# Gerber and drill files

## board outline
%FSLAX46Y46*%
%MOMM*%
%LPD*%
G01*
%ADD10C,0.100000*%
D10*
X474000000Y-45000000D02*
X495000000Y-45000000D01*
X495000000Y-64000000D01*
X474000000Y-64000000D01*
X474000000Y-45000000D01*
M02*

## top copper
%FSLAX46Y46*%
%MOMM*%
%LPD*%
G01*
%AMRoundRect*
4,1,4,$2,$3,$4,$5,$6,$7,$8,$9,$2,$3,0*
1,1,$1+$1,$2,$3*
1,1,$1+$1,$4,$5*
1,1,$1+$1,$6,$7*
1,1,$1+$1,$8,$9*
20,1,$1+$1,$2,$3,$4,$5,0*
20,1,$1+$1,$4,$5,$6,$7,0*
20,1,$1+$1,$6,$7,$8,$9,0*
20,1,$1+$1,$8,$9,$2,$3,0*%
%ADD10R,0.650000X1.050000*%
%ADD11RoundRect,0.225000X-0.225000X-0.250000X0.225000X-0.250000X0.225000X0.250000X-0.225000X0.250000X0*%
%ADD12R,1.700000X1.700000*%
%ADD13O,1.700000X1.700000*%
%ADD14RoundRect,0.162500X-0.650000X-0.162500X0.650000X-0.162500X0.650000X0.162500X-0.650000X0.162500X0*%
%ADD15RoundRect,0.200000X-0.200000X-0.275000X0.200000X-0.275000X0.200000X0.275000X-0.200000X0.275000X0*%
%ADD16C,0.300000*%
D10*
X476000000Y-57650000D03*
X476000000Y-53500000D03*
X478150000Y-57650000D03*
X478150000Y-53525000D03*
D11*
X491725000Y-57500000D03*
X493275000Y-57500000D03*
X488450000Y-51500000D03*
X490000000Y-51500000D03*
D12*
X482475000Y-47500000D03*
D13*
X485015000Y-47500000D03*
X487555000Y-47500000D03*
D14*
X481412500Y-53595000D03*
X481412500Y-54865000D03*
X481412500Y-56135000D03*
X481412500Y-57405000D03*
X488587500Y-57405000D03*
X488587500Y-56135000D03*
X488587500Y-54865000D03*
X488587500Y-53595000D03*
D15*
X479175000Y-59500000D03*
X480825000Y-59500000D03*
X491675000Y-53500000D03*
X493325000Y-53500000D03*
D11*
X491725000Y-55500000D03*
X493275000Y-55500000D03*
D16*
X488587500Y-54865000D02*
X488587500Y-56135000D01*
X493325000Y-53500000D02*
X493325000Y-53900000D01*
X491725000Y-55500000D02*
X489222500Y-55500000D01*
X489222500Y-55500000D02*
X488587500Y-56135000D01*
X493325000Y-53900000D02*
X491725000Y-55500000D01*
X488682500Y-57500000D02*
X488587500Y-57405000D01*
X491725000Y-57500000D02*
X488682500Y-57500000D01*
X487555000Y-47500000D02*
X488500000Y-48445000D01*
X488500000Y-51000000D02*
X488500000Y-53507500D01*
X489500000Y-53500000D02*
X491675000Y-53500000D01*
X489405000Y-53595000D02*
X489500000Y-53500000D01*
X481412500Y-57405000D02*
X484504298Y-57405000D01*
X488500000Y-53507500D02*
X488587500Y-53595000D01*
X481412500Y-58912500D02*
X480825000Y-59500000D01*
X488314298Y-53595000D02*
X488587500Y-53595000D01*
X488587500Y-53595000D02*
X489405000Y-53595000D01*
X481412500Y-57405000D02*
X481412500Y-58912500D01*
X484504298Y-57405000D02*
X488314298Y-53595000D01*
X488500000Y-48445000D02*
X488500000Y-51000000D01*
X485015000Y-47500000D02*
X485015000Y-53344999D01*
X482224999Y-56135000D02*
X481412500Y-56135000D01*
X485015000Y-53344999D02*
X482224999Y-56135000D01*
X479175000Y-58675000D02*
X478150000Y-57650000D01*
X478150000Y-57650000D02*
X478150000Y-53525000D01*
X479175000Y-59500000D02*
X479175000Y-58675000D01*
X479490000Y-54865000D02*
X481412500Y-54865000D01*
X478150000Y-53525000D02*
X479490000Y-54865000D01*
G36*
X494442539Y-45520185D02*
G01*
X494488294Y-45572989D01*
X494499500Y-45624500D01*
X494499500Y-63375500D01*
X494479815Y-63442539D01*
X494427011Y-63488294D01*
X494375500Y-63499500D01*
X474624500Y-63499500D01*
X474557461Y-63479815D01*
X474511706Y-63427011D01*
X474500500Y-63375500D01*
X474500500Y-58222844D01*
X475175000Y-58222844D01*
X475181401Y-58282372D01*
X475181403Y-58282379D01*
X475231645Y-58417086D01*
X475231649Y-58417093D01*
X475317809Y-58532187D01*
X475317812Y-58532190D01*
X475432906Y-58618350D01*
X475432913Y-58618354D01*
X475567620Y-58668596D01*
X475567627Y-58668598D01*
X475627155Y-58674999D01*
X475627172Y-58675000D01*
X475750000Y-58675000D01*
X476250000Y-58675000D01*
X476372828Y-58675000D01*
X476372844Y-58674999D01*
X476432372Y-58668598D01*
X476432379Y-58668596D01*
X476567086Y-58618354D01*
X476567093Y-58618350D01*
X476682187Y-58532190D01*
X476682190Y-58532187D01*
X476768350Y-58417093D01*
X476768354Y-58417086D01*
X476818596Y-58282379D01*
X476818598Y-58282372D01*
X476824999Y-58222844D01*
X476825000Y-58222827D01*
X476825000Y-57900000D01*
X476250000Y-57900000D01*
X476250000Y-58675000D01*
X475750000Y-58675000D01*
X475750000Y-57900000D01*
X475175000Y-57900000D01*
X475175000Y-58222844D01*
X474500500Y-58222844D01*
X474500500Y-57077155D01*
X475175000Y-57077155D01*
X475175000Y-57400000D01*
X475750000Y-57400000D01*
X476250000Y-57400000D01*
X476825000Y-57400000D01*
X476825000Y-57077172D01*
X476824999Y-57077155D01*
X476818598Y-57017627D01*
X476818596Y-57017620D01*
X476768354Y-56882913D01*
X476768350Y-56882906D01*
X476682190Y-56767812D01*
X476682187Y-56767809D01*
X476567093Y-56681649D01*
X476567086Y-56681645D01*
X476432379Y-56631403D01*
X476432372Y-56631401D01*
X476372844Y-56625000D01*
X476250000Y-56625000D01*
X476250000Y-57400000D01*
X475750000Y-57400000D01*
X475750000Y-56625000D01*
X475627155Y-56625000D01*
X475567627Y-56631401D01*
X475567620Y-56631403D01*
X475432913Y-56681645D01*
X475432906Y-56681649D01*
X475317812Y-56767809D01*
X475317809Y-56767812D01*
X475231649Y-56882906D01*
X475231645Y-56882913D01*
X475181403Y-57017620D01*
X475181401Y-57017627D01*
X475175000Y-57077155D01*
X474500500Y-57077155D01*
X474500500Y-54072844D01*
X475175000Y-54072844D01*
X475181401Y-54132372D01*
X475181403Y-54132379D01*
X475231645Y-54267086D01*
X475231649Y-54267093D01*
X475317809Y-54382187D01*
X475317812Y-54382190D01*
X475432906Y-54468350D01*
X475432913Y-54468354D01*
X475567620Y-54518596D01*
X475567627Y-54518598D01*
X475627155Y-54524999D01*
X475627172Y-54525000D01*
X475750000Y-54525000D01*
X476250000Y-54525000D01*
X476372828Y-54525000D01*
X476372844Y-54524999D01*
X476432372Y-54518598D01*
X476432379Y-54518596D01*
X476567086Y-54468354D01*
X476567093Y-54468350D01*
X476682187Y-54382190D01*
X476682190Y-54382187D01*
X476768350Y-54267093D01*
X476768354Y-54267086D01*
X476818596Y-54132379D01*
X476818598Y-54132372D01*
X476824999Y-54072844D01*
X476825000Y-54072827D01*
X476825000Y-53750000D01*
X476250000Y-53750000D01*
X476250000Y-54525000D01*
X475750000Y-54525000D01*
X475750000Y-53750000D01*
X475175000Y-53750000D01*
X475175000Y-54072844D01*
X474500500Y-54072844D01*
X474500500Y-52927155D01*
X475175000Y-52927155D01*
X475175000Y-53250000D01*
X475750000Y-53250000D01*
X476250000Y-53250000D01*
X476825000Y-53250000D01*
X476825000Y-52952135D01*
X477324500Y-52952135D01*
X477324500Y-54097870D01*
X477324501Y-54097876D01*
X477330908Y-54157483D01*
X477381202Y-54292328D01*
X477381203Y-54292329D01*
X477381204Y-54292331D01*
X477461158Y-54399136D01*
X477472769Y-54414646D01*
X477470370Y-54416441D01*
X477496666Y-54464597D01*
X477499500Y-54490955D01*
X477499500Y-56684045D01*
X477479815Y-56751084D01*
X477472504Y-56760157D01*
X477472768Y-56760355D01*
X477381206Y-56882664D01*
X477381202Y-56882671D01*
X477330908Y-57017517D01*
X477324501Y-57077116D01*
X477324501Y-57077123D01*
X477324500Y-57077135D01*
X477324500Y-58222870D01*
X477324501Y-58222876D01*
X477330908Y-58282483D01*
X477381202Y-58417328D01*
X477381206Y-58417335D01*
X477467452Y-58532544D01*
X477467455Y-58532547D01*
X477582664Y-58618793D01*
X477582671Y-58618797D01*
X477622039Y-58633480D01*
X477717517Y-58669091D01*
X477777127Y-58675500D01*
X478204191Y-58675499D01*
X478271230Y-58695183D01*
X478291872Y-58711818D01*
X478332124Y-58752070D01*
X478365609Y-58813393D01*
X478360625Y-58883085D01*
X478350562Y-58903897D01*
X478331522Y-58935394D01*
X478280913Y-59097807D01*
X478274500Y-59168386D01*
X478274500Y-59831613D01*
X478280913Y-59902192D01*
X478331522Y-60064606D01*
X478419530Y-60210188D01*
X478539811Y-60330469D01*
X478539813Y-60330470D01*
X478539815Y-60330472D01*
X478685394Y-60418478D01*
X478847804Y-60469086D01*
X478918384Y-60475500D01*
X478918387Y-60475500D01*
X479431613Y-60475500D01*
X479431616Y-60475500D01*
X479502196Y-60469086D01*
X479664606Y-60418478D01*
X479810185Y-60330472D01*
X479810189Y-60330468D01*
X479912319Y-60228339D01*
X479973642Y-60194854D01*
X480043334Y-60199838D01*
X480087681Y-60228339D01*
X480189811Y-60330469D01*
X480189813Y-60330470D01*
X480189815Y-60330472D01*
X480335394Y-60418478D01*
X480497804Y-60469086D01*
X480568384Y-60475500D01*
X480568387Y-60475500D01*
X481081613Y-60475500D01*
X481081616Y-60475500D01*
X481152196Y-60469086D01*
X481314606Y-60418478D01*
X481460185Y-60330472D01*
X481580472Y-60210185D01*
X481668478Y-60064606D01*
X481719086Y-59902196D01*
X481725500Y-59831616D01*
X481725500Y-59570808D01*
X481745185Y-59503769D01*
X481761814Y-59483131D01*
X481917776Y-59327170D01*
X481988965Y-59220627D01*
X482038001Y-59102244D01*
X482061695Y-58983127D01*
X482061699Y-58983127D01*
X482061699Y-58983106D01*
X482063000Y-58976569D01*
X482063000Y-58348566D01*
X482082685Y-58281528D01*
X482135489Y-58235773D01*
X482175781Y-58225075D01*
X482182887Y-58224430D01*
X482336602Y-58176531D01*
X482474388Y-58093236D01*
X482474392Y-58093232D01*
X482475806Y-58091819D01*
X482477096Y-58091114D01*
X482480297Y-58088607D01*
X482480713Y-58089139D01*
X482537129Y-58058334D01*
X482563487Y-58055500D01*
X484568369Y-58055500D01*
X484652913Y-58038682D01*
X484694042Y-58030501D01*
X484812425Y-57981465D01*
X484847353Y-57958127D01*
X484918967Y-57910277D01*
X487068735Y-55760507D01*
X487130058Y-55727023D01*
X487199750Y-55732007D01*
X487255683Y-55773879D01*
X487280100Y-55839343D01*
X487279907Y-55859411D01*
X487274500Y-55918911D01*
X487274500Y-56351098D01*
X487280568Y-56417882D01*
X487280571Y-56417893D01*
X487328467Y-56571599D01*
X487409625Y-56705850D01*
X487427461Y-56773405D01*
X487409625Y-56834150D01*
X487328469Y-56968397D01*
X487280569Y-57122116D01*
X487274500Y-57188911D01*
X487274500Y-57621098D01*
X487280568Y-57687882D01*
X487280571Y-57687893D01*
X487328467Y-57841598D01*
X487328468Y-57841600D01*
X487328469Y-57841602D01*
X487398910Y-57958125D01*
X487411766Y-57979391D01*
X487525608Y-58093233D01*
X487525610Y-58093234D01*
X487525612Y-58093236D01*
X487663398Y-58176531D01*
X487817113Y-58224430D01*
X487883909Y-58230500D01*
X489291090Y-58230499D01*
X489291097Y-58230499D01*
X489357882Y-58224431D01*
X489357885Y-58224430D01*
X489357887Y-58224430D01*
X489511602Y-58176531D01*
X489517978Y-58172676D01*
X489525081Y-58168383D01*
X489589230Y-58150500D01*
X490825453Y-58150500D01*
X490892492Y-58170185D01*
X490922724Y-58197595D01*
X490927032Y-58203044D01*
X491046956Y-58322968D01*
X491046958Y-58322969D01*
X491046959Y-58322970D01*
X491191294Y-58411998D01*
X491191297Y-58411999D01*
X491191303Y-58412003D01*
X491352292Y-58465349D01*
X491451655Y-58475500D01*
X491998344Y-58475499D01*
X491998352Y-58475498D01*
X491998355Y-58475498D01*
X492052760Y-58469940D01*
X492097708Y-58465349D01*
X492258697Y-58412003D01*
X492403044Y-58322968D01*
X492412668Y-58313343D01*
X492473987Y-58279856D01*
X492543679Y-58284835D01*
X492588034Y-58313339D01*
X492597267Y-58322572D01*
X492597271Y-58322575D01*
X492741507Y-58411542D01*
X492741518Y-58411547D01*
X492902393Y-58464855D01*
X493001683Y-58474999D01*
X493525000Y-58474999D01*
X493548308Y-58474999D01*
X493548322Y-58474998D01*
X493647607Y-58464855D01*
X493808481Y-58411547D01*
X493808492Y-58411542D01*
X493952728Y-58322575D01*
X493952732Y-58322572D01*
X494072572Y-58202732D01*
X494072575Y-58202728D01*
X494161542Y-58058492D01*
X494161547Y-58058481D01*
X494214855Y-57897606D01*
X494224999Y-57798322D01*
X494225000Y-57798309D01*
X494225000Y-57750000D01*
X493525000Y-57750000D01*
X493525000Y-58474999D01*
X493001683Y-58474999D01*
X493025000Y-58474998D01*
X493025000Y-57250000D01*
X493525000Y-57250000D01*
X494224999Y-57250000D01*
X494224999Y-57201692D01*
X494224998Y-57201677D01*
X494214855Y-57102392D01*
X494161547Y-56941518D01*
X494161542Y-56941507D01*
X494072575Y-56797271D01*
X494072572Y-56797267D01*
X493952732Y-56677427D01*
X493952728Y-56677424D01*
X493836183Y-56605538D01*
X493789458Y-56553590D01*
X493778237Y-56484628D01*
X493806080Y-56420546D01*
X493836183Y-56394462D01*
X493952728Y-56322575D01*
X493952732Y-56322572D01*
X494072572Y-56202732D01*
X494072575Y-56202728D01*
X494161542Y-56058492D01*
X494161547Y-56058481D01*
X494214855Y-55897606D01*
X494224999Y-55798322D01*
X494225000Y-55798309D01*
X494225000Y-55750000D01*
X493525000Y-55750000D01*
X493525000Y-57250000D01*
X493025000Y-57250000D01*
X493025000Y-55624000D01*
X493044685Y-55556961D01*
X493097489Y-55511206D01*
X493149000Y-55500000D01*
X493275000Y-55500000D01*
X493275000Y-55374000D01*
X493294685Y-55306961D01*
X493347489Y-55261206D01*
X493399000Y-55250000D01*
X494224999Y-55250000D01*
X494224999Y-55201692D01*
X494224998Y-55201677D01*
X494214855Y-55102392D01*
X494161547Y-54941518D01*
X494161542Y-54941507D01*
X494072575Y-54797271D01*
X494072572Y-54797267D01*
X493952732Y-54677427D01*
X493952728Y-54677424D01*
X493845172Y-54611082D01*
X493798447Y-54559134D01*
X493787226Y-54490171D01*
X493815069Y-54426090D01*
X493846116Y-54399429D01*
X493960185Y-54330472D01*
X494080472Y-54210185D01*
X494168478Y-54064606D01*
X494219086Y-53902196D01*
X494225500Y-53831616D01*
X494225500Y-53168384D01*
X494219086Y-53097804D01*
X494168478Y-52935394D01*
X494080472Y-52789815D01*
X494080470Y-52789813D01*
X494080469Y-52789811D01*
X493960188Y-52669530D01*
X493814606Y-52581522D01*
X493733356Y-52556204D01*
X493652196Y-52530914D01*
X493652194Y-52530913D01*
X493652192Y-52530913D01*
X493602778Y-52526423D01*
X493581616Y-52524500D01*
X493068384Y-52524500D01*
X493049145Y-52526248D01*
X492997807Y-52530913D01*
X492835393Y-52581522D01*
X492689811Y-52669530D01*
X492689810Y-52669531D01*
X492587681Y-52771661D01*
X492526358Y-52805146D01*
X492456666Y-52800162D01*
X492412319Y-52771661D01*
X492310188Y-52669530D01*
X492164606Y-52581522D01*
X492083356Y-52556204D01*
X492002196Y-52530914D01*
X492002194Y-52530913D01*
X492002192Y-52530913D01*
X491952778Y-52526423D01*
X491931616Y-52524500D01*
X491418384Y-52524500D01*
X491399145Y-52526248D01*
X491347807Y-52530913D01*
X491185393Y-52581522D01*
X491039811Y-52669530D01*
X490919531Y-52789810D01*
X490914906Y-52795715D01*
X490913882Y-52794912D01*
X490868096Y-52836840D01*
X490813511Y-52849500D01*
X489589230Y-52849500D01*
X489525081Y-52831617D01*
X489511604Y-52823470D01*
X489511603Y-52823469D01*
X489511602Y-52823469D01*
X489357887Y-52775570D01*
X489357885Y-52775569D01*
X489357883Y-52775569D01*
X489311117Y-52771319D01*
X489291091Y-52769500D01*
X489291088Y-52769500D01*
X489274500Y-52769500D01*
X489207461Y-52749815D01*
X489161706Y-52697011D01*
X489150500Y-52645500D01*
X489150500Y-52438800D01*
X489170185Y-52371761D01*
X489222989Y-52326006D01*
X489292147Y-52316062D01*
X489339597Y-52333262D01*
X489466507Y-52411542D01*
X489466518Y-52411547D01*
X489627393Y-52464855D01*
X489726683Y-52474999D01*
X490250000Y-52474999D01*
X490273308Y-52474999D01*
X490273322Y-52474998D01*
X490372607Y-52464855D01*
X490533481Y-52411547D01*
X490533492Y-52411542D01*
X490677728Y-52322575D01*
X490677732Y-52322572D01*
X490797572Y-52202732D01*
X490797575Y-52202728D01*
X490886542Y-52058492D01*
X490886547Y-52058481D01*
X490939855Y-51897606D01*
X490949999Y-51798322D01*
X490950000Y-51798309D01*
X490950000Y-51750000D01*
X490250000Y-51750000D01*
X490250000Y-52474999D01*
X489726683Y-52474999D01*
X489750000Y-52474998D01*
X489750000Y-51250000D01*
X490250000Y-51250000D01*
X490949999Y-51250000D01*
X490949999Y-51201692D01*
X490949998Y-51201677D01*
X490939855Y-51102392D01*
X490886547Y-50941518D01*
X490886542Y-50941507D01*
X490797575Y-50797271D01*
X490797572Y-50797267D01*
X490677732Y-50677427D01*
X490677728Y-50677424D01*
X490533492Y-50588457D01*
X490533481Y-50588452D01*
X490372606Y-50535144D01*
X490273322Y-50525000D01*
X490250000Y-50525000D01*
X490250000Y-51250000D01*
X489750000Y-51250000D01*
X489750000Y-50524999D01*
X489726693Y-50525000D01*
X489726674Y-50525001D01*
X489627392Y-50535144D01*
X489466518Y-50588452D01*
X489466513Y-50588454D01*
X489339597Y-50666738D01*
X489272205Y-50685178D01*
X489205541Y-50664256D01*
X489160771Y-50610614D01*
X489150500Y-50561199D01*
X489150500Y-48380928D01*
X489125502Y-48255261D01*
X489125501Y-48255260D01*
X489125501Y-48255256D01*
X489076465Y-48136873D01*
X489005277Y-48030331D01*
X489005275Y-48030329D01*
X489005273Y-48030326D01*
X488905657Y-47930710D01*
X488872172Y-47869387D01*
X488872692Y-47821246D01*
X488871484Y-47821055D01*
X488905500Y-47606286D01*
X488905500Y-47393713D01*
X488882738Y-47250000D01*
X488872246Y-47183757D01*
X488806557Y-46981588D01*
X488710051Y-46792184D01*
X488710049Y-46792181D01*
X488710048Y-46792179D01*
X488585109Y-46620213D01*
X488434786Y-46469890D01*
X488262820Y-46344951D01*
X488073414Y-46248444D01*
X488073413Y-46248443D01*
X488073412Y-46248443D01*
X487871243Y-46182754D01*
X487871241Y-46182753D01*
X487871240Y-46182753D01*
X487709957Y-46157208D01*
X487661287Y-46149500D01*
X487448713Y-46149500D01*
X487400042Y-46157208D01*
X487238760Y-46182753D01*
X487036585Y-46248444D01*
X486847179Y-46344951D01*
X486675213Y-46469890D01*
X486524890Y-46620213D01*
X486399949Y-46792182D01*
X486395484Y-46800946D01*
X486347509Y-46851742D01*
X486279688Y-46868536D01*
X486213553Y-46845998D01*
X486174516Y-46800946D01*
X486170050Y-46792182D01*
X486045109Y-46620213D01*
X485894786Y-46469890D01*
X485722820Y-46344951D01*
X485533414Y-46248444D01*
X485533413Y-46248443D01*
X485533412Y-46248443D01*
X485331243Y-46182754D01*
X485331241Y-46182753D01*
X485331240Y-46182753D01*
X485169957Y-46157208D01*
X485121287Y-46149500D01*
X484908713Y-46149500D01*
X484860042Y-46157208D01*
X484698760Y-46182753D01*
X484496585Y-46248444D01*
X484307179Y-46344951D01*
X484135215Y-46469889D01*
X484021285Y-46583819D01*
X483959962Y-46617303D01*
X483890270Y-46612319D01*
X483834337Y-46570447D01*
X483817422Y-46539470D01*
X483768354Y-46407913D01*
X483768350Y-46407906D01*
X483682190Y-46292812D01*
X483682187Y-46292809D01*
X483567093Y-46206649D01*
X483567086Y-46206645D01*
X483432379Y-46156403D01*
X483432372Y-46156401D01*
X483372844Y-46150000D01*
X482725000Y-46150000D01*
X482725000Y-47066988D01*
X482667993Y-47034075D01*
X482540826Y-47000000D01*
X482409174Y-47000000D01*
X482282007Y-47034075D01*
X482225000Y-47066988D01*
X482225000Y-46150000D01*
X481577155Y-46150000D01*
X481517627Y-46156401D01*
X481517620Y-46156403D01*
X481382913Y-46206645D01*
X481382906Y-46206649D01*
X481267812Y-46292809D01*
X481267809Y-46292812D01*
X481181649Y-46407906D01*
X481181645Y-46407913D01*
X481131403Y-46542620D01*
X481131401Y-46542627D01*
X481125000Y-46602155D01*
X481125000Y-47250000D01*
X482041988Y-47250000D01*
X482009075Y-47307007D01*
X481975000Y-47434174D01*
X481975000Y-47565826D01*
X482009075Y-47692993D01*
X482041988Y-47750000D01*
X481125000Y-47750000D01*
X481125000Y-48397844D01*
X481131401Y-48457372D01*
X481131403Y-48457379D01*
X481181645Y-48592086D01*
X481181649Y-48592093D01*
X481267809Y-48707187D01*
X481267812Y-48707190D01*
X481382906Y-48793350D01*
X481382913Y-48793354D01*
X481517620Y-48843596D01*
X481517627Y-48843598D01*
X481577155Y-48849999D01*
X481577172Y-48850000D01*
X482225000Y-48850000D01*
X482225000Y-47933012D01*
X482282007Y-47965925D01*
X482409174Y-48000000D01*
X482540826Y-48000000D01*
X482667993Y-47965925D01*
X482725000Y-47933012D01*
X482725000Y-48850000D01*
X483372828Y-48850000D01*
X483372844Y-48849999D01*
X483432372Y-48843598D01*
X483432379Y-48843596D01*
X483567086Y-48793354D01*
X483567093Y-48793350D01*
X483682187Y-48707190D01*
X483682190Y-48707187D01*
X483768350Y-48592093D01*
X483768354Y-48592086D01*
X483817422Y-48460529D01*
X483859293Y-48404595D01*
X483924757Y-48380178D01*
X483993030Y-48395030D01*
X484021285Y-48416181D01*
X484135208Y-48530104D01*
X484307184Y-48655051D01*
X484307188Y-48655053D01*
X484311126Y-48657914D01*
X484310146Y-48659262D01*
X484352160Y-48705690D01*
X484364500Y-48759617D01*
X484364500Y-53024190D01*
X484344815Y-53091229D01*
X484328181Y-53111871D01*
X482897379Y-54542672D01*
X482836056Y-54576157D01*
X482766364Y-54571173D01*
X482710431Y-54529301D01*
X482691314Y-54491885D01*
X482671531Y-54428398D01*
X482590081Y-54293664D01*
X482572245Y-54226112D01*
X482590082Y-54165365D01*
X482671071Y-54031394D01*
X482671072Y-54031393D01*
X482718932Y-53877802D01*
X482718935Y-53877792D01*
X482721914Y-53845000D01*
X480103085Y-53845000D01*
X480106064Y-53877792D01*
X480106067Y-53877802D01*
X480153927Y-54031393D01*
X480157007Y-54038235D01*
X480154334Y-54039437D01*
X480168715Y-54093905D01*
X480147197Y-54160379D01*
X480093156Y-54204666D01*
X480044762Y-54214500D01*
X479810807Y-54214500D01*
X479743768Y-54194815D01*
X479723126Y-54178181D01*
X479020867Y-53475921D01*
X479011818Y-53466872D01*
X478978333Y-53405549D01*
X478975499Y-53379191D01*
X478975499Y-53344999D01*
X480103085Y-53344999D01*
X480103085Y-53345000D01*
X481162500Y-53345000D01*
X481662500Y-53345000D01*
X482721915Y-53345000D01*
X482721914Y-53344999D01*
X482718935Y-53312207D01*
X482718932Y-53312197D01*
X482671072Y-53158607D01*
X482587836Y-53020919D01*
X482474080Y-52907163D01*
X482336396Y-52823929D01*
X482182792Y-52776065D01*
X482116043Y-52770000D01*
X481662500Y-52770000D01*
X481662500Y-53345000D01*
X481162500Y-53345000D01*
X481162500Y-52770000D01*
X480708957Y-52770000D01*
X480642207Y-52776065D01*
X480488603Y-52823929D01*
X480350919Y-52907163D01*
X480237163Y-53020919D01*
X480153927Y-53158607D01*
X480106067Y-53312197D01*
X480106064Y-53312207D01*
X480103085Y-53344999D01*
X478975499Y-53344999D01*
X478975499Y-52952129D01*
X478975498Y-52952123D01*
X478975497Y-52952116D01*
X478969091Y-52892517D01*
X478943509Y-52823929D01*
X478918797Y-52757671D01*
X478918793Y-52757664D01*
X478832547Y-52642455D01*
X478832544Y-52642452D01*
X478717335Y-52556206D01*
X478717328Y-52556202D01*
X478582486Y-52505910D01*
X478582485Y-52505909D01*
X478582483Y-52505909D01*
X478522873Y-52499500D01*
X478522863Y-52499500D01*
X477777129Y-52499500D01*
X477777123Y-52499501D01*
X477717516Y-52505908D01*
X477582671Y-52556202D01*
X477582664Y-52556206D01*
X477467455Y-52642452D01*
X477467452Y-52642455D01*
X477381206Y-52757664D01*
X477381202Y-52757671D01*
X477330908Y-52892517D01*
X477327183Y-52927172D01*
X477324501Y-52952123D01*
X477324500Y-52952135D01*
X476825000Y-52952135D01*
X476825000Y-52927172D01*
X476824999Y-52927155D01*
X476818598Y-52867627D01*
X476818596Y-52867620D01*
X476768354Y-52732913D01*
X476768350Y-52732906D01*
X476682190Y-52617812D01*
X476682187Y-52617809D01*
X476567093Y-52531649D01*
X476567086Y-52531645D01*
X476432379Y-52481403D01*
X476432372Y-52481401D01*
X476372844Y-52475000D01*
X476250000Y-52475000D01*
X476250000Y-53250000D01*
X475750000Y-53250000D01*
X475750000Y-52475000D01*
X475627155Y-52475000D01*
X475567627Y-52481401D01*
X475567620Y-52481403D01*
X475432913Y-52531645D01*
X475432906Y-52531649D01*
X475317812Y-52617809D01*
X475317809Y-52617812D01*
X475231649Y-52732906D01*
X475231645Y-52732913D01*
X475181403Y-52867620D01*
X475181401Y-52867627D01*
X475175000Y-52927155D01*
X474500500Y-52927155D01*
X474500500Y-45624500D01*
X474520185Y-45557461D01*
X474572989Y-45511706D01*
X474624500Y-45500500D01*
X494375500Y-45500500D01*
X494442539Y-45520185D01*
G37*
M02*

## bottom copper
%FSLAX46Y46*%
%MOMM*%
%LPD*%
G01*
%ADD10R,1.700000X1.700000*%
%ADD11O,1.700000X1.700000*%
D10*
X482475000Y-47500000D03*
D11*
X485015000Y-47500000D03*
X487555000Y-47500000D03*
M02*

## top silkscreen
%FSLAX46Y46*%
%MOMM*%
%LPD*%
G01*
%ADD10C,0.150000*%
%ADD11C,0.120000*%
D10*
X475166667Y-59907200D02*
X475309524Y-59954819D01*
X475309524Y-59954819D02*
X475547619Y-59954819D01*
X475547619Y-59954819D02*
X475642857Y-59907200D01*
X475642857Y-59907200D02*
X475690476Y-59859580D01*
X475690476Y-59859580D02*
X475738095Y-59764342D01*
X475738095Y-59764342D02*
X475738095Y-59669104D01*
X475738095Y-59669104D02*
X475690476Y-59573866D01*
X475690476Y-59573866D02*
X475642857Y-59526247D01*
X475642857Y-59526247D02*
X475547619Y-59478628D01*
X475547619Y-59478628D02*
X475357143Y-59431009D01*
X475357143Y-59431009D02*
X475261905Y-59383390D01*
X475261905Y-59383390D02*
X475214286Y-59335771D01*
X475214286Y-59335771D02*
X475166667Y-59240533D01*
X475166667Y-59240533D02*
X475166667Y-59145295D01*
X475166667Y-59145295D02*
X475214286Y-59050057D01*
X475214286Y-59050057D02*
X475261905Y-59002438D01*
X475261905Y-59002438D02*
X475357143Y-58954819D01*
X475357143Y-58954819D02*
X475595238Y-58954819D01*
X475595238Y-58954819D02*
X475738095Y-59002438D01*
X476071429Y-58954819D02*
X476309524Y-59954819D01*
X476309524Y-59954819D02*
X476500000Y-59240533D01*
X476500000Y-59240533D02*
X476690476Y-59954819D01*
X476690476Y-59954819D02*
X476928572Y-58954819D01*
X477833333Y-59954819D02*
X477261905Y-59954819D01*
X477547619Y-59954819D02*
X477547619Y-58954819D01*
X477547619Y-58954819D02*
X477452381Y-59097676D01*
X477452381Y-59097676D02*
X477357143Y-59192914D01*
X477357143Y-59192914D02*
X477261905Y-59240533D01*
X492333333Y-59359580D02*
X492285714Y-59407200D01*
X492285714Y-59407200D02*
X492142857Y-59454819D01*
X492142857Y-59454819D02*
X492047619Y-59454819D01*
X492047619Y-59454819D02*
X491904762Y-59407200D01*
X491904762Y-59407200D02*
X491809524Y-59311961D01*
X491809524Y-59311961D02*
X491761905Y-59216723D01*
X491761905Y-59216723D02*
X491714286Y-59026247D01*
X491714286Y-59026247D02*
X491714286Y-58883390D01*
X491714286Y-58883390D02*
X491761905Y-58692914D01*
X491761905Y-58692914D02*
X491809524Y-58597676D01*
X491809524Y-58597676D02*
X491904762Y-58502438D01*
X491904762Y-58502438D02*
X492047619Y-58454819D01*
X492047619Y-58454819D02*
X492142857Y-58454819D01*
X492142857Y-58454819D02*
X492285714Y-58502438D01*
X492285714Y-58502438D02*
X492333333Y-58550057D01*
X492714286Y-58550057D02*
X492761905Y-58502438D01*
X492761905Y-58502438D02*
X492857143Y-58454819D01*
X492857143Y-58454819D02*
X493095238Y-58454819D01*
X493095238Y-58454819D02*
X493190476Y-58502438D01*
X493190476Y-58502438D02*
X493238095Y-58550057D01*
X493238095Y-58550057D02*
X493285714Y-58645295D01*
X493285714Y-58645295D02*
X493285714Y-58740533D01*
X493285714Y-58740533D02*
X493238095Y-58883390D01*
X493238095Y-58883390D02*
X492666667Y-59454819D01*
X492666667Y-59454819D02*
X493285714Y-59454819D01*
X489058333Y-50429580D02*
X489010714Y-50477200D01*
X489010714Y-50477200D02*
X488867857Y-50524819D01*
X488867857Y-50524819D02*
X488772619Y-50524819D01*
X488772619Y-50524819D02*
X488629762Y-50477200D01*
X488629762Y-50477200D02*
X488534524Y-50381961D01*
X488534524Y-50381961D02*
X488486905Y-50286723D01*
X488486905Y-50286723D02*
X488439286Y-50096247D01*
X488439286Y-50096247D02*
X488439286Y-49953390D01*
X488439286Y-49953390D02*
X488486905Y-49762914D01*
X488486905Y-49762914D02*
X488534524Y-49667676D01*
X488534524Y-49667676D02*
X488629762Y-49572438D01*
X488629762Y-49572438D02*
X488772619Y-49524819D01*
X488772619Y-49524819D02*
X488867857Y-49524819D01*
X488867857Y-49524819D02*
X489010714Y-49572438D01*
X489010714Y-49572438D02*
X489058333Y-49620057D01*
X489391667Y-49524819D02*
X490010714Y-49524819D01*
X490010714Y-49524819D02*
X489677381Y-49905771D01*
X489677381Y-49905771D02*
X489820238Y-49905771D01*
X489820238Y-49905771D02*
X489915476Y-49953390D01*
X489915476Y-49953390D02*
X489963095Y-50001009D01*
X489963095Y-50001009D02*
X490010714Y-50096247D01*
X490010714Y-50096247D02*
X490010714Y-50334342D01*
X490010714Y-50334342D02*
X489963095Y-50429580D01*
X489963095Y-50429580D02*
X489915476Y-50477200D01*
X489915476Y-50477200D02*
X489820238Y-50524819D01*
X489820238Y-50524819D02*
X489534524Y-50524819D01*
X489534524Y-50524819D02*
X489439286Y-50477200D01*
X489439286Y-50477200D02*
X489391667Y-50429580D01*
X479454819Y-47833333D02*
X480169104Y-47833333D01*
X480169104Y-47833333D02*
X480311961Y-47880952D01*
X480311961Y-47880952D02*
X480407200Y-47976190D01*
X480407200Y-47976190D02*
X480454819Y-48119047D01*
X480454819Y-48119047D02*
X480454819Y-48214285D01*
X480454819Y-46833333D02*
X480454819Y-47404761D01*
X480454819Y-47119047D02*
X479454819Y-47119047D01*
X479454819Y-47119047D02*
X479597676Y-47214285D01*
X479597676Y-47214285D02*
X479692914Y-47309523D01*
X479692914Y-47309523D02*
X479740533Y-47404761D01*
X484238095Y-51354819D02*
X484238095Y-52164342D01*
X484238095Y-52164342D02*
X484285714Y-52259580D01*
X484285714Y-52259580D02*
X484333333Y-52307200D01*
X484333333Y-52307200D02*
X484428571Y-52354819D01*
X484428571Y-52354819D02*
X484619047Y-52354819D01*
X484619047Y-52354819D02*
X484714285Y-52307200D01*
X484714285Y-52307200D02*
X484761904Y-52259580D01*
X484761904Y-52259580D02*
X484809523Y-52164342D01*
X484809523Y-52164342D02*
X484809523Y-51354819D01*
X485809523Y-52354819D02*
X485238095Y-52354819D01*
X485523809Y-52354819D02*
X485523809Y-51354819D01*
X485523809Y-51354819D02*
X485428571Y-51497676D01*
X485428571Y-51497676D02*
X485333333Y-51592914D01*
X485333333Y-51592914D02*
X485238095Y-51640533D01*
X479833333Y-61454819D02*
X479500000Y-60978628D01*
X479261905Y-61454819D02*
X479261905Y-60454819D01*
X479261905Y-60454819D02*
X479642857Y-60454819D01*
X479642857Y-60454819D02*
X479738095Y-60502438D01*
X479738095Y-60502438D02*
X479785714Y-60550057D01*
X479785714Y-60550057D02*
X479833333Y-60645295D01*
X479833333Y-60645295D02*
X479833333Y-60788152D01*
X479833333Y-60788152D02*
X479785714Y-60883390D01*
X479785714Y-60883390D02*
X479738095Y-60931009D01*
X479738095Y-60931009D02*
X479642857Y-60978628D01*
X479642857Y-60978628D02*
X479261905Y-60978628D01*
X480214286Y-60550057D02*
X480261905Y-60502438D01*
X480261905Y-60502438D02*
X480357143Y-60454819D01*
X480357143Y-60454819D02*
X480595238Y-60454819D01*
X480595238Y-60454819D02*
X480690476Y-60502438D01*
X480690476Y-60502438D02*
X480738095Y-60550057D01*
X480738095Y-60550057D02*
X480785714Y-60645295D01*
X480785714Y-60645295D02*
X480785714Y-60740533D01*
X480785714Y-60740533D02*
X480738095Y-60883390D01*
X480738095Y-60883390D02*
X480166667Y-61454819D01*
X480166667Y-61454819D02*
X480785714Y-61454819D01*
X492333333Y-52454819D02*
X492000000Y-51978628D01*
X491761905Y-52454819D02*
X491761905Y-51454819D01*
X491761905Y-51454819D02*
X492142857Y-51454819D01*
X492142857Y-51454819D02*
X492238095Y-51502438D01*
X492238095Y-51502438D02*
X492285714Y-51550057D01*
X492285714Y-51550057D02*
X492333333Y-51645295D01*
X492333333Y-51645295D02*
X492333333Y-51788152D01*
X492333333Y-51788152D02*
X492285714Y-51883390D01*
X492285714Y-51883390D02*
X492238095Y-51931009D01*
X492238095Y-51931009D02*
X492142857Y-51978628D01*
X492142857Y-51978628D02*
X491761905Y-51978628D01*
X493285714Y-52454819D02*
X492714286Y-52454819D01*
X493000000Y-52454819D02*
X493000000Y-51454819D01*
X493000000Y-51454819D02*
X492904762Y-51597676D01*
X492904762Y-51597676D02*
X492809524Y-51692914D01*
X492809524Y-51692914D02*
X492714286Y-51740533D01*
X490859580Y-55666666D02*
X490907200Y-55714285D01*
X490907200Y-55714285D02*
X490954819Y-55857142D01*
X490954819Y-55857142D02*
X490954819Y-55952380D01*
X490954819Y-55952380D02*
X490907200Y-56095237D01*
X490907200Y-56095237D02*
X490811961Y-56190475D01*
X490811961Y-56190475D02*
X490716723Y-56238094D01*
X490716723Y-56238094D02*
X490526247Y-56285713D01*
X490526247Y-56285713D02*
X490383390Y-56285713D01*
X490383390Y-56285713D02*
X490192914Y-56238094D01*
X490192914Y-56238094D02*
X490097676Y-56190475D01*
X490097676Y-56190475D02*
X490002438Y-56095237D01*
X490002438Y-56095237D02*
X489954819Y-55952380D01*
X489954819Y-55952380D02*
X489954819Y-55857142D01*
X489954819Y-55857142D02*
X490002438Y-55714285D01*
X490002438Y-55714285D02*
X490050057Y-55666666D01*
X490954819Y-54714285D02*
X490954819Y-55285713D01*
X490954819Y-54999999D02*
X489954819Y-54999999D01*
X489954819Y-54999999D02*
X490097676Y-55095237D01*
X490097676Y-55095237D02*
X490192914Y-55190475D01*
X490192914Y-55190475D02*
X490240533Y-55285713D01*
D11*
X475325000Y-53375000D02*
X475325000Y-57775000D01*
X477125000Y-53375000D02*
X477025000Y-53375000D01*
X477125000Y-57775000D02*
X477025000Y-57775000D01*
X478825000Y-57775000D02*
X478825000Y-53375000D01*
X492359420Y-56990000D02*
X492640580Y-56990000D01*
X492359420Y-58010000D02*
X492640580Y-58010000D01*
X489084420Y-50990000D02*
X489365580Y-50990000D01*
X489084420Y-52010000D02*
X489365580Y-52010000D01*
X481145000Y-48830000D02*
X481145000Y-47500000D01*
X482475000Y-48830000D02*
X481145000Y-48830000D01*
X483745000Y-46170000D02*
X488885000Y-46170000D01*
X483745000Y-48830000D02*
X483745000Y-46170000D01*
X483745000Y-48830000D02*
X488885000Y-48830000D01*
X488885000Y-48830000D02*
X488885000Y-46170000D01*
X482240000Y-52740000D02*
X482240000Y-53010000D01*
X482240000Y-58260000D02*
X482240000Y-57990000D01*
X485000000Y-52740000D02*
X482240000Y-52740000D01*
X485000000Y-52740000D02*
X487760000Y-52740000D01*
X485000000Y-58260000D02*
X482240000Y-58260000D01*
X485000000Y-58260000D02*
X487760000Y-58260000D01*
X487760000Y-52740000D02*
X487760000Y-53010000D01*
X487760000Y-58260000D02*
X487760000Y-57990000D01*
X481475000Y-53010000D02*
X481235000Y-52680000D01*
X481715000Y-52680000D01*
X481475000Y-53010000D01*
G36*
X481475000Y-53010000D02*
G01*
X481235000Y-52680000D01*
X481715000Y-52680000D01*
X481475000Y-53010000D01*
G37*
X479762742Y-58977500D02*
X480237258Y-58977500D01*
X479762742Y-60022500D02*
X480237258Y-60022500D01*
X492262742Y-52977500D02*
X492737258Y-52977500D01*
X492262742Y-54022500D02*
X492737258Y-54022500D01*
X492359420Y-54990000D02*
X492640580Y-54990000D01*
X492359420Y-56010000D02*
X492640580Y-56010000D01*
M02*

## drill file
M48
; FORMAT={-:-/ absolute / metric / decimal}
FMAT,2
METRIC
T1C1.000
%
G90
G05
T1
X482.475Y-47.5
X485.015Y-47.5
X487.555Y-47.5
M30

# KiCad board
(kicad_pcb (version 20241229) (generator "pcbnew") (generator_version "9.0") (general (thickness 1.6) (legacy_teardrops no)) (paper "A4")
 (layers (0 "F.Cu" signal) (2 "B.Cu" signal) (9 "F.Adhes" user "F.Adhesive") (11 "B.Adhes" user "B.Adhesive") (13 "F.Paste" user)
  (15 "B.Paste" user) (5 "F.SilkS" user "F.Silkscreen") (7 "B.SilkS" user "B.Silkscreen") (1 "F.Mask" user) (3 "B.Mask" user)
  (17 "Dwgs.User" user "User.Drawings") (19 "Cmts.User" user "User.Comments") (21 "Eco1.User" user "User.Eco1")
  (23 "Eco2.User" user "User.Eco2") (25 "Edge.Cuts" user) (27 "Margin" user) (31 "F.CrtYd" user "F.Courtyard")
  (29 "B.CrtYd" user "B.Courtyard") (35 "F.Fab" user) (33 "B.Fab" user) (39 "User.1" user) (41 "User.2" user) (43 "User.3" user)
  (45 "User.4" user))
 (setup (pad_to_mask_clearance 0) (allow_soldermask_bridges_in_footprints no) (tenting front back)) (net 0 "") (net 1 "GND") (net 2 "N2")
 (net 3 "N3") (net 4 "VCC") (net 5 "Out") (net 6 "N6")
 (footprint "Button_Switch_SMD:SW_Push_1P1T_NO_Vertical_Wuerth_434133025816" (layer "F.Cu") (at 477.075 55.575 90)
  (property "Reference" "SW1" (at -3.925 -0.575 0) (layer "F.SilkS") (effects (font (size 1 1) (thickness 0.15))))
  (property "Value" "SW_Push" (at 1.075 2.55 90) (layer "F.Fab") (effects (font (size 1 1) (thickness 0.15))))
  (fp_line (start 2.2 -1.75) (end -2.2 -1.75) (stroke (width 0.12) (type solid)) (layer "F.SilkS"))
  (fp_line (start 2.2 0.05) (end 2.2 -0.05) (stroke (width 0.12) (type solid)) (layer "F.SilkS"))
  (fp_line (start -2.2 0.05) (end -2.2 -0.05) (stroke (width 0.12) (type solid)) (layer "F.SilkS"))
  (fp_line (start -2.2 1.75) (end 2.2 1.75) (stroke (width 0.12) (type solid)) (layer "F.SilkS"))
  (pad "1" smd rect (at -2.075 -1.075 90) (size 1.05 0.65) (layers "F.Cu" "F.Mask" "F.Paste") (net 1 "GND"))
  (pad "1" smd rect (at 2.075 -1.075 90) (size 1.05 0.65) (layers "F.Cu" "F.Mask" "F.Paste") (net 1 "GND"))
  (pad "2" smd rect (at -2.075 1.075 90) (size 1.05 0.65) (layers "F.Cu" "F.Mask" "F.Paste") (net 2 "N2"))
  (pad "2" smd rect (at 2.05 1.075 90) (size 1.05 0.65) (layers "F.Cu" "F.Mask" "F.Paste") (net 2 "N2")))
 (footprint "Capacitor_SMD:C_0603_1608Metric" (layer "F.Cu") (at 492.5 57.5)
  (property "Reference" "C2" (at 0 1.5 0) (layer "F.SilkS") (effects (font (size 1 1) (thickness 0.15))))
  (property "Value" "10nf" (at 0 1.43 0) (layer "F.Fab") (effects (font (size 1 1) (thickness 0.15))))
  (fp_line (start -0.14058 -0.51) (end 0.14058 -0.51) (stroke (width 0.12) (type solid)) (layer "F.SilkS"))
  (fp_line (start -0.14058 0.51) (end 0.14058 0.51) (stroke (width 0.12) (type solid)) (layer "F.SilkS"))
  (pad "1" smd roundrect (at -0.775 0) (size 0.9 0.95) (layers "F.Cu" "F.Mask" "F.Paste") (roundrect_rratio 0.25) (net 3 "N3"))
  (pad "2" smd roundrect (at 0.775 0) (size 0.9 0.95) (layers "F.Cu" "F.Mask" "F.Paste") (roundrect_rratio 0.25) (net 1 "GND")))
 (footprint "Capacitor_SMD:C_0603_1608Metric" (layer "F.Cu") (at 489.225 51.5)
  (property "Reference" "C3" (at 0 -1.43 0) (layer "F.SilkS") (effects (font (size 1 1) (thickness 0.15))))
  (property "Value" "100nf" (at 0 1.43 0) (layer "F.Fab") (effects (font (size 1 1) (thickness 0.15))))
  (fp_line (start -0.14058 -0.51) (end 0.14058 -0.51) (stroke (width 0.12) (type solid)) (layer "F.SilkS"))
  (fp_line (start -0.14058 0.51) (end 0.14058 0.51) (stroke (width 0.12) (type solid)) (layer "F.SilkS"))
  (pad "1" smd roundrect (at -0.775 0) (size 0.9 0.95) (layers "F.Cu" "F.Mask" "F.Paste") (roundrect_rratio 0.25) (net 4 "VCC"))
  (pad "2" smd roundrect (at 0.775 0) (size 0.9 0.95) (layers "F.Cu" "F.Mask" "F.Paste") (roundrect_rratio 0.25) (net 1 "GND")))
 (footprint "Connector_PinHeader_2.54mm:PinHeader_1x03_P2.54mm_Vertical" (layer "F.Cu") (at 482.475 47.5 90)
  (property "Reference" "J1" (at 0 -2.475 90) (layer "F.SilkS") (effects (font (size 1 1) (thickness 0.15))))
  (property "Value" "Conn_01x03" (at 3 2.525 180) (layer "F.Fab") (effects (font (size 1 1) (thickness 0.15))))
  (fp_line (start -1.33 -1.33) (end 0 -1.33) (stroke (width 0.12) (type solid)) (layer "F.SilkS"))
  (fp_line (start -1.33 0) (end -1.33 -1.33) (stroke (width 0.12) (type solid)) (layer "F.SilkS"))
  (fp_line (start 1.33 1.27) (end 1.33 6.41) (stroke (width 0.12) (type solid)) (layer "F.SilkS"))
  (fp_line (start -1.33 1.27) (end 1.33 1.27) (stroke (width 0.12) (type solid)) (layer "F.SilkS"))
  (fp_line (start -1.33 1.27) (end -1.33 6.41) (stroke (width 0.12) (type solid)) (layer "F.SilkS"))
  (fp_line (start -1.33 6.41) (end 1.33 6.41) (stroke (width 0.12) (type solid)) (layer "F.SilkS"))
  (pad "1" thru_hole rect (at 0 0 90) (size 1.7 1.7) (drill 1) (layers "*.Cu" "*.Mask") (remove_unused_layers no) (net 1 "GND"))
  (pad "2" thru_hole oval (at 0 2.54 90) (size 1.7 1.7) (drill 1) (layers "*.Cu" "*.Mask") (remove_unused_layers no) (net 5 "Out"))
  (pad "3" thru_hole oval (at 0 5.08 90) (size 1.7 1.7) (drill 1) (layers "*.Cu" "*.Mask") (remove_unused_layers no) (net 4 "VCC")))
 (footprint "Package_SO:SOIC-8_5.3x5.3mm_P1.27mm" (layer "F.Cu") (at 485 55.5)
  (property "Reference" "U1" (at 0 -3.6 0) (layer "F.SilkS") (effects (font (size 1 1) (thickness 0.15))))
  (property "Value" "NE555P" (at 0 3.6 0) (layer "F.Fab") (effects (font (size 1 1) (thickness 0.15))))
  (fp_line (start -2.76 -2.76) (end -2.76 -2.49) (stroke (width 0.12) (type solid)) (layer "F.SilkS"))
  (fp_line (start -2.76 2.76) (end -2.76 2.49) (stroke (width 0.12) (type solid)) (layer "F.SilkS"))
  (fp_line (start 0 -2.76) (end -2.76 -2.76) (stroke (width 0.12) (type solid)) (layer "F.SilkS"))
  (fp_line (start 0 -2.76) (end 2.76 -2.76) (stroke (width 0.12) (type solid)) (layer "F.SilkS"))
  (fp_line (start 0 2.76) (end -2.76 2.76) (stroke (width 0.12) (type solid)) (layer "F.SilkS"))
  (fp_line (start 0 2.76) (end 2.76 2.76) (stroke (width 0.12) (type solid)) (layer "F.SilkS"))
  (fp_line (start 2.76 -2.76) (end 2.76 -2.49) (stroke (width 0.12) (type solid)) (layer "F.SilkS"))
  (fp_line (start 2.76 2.76) (end 2.76 2.49) (stroke (width 0.12) (type solid)) (layer "F.SilkS"))
  (fp_poly
   (pts (xy -3.525 -2.49) (xy -3.765 -2.82) (xy -3.285 -2.82) (xy -3.525 -2.49)) (stroke (width 0.12) (type solid)) (fill yes)
   (layer "F.SilkS"))
  (pad "1" smd roundrect (at -3.5875 -1.905) (size 1.625 0.65) (layers "F.Cu" "F.Mask" "F.Paste") (roundrect_rratio 0.25) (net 1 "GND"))
  (pad "2" smd roundrect (at -3.5875 -0.635) (size 1.625 0.65) (layers "F.Cu" "F.Mask" "F.Paste") (roundrect_rratio 0.25) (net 2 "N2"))
  (pad "3" smd roundrect (at -3.5875 0.635) (size 1.625 0.65) (layers "F.Cu" "F.Mask" "F.Paste") (roundrect_rratio 0.25) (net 5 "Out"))
  (pad "4" smd roundrect (at -3.5875 1.905) (size 1.625 0.65) (layers "F.Cu" "F.Mask" "F.Paste") (roundrect_rratio 0.25) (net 4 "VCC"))
  (pad "5" smd roundrect (at 3.5875 1.905) (size 1.625 0.65) (layers "F.Cu" "F.Mask" "F.Paste") (roundrect_rratio 0.25) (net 3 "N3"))
  (pad "6" smd roundrect (at 3.5875 0.635) (size 1.625 0.65) (layers "F.Cu" "F.Mask" "F.Paste") (roundrect_rratio 0.25) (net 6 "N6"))
  (pad "7" smd roundrect (at 3.5875 -0.635) (size 1.625 0.65) (layers "F.Cu" "F.Mask" "F.Paste") (roundrect_rratio 0.25) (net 6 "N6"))
  (pad "8" smd roundrect (at 3.5875 -1.905) (size 1.625 0.65) (layers "F.Cu" "F.Mask" "F.Paste") (roundrect_rratio 0.25) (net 4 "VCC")))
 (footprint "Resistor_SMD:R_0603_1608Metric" (layer "F.Cu") (at 480 59.5)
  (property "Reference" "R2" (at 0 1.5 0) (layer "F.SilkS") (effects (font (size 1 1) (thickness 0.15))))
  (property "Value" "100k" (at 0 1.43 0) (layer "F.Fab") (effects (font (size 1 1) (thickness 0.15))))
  (fp_line (start -0.237258 -0.5225) (end 0.237258 -0.5225) (stroke (width 0.12) (type solid)) (layer "F.SilkS"))
  (fp_line (start -0.237258 0.5225) (end 0.237258 0.5225) (stroke (width 0.12) (type solid)) (layer "F.SilkS"))
  (pad "1" smd roundrect (at -0.825 0) (size 0.8 0.95) (layers "F.Cu" "F.Mask" "F.Paste") (roundrect_rratio 0.25) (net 2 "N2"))
  (pad "2" smd roundrect (at 0.825 0) (size 0.8 0.95) (layers "F.Cu" "F.Mask" "F.Paste") (roundrect_rratio 0.25) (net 4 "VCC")))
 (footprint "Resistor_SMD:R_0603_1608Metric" (layer "F.Cu") (at 492.5 53.5)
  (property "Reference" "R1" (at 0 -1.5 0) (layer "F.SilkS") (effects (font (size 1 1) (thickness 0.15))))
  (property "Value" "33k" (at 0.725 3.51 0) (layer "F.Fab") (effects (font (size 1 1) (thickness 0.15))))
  (fp_line (start -0.237258 -0.5225) (end 0.237258 -0.5225) (stroke (width 0.12) (type solid)) (layer "F.SilkS"))
  (fp_line (start -0.237258 0.5225) (end 0.237258 0.5225) (stroke (width 0.12) (type solid)) (layer "F.SilkS"))
  (pad "1" smd roundrect (at -0.825 0) (size 0.8 0.95) (layers "F.Cu" "F.Mask" "F.Paste") (roundrect_rratio 0.25) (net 4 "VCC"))
  (pad "2" smd roundrect (at 0.825 0) (size 0.8 0.95) (layers "F.Cu" "F.Mask" "F.Paste") (roundrect_rratio 0.25) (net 6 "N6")))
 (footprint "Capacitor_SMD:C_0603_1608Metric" (layer "F.Cu") (at 492.5 55.5)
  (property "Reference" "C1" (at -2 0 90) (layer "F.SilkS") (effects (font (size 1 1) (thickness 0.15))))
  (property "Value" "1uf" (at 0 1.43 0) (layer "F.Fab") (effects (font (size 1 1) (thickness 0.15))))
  (fp_line (start -0.14058 -0.51) (end 0.14058 -0.51) (stroke (width 0.12) (type solid)) (layer "F.SilkS"))
  (fp_line (start -0.14058 0.51) (end 0.14058 0.51) (stroke (width 0.12) (type solid)) (layer "F.SilkS"))
  (pad "1" smd roundrect (at -0.775 0) (size 0.9 0.95) (layers "F.Cu" "F.Mask" "F.Paste") (roundrect_rratio 0.25) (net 6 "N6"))
  (pad "2" smd roundrect (at 0.775 0) (size 0.9 0.95) (layers "F.Cu" "F.Mask" "F.Paste") (roundrect_rratio 0.25) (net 1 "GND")))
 (gr_rect (start 474 45) (end 495 64) (stroke (width 0.1) (type solid)) (fill no) (layer "Edge.Cuts"))
 (segment (start 488.5875 54.865) (end 488.5875 56.135) (width 0.3) (layer "F.Cu") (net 6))
 (segment (start 493.325 53.5) (end 493.325 53.9) (width 0.3) (layer "F.Cu") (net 6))
 (segment (start 491.725 55.5) (end 489.2225 55.5) (width 0.3) (layer "F.Cu") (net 6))
 (segment (start 489.2225 55.5) (end 488.5875 56.135) (width 0.3) (layer "F.Cu") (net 6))
 (segment (start 493.325 53.9) (end 491.725 55.5) (width 0.3) (layer "F.Cu") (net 6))
 (segment (start 488.6825 57.5) (end 488.5875 57.405) (width 0.3) (layer "F.Cu") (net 3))
 (segment (start 491.725 57.5) (end 488.6825 57.5) (width 0.3) (layer "F.Cu") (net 3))
 (segment (start 487.555 47.5) (end 488.5 48.445) (width 0.3) (layer "F.Cu") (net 4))
 (segment (start 488.5 51) (end 488.5 53.5075) (width 0.3) (layer "F.Cu") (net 4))
 (segment (start 489.5 53.5) (end 491.675 53.5) (width 0.3) (layer "F.Cu") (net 4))
 (segment (start 489.405 53.595) (end 489.5 53.5) (width 0.3) (layer "F.Cu") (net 4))
 (segment (start 481.4125 57.405) (end 484.504298 57.405) (width 0.3) (layer "F.Cu") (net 4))
 (segment (start 488.5 53.5075) (end 488.5875 53.595) (width 0.3) (layer "F.Cu") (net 4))
 (segment (start 481.4125 58.9125) (end 480.825 59.5) (width 0.3) (layer "F.Cu") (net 4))
 (segment (start 488.314298 53.595) (end 488.5875 53.595) (width 0.3) (layer "F.Cu") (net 4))
 (segment (start 488.5875 53.595) (end 489.405 53.595) (width 0.3) (layer "F.Cu") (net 4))
 (segment (start 481.4125 57.405) (end 481.4125 58.9125) (width 0.3) (layer "F.Cu") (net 4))
 (segment (start 484.504298 57.405) (end 488.314298 53.595) (width 0.3) (layer "F.Cu") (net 4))
 (segment (start 488.5 48.445) (end 488.5 51) (width 0.3) (layer "F.Cu") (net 4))
 (segment (start 485.015 47.5) (end 485.015 53.344999) (width 0.3) (layer "F.Cu") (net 5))
 (segment (start 482.224999 56.135) (end 481.4125 56.135) (width 0.3) (layer "F.Cu") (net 5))
 (segment (start 485.015 53.344999) (end 482.224999 56.135) (width 0.3) (layer "F.Cu") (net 5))
 (segment (start 479.175 58.675) (end 478.15 57.65) (width 0.3) (layer "F.Cu") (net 2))
 (segment (start 478.15 57.65) (end 478.15 53.525) (width 0.3) (layer "F.Cu") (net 2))
 (segment (start 479.175 59.5) (end 479.175 58.675) (width 0.3) (layer "F.Cu") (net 2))
 (segment (start 479.49 54.865) (end 481.4125 54.865) (width 0.3) (layer "F.Cu") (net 2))
 (segment (start 478.15 53.525) (end 479.49 54.865) (width 0.3) (layer "F.Cu") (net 2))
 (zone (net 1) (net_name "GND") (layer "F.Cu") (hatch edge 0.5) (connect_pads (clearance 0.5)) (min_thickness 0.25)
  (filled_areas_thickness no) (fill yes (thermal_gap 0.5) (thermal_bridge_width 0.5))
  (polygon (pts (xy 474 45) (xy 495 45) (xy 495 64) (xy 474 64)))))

